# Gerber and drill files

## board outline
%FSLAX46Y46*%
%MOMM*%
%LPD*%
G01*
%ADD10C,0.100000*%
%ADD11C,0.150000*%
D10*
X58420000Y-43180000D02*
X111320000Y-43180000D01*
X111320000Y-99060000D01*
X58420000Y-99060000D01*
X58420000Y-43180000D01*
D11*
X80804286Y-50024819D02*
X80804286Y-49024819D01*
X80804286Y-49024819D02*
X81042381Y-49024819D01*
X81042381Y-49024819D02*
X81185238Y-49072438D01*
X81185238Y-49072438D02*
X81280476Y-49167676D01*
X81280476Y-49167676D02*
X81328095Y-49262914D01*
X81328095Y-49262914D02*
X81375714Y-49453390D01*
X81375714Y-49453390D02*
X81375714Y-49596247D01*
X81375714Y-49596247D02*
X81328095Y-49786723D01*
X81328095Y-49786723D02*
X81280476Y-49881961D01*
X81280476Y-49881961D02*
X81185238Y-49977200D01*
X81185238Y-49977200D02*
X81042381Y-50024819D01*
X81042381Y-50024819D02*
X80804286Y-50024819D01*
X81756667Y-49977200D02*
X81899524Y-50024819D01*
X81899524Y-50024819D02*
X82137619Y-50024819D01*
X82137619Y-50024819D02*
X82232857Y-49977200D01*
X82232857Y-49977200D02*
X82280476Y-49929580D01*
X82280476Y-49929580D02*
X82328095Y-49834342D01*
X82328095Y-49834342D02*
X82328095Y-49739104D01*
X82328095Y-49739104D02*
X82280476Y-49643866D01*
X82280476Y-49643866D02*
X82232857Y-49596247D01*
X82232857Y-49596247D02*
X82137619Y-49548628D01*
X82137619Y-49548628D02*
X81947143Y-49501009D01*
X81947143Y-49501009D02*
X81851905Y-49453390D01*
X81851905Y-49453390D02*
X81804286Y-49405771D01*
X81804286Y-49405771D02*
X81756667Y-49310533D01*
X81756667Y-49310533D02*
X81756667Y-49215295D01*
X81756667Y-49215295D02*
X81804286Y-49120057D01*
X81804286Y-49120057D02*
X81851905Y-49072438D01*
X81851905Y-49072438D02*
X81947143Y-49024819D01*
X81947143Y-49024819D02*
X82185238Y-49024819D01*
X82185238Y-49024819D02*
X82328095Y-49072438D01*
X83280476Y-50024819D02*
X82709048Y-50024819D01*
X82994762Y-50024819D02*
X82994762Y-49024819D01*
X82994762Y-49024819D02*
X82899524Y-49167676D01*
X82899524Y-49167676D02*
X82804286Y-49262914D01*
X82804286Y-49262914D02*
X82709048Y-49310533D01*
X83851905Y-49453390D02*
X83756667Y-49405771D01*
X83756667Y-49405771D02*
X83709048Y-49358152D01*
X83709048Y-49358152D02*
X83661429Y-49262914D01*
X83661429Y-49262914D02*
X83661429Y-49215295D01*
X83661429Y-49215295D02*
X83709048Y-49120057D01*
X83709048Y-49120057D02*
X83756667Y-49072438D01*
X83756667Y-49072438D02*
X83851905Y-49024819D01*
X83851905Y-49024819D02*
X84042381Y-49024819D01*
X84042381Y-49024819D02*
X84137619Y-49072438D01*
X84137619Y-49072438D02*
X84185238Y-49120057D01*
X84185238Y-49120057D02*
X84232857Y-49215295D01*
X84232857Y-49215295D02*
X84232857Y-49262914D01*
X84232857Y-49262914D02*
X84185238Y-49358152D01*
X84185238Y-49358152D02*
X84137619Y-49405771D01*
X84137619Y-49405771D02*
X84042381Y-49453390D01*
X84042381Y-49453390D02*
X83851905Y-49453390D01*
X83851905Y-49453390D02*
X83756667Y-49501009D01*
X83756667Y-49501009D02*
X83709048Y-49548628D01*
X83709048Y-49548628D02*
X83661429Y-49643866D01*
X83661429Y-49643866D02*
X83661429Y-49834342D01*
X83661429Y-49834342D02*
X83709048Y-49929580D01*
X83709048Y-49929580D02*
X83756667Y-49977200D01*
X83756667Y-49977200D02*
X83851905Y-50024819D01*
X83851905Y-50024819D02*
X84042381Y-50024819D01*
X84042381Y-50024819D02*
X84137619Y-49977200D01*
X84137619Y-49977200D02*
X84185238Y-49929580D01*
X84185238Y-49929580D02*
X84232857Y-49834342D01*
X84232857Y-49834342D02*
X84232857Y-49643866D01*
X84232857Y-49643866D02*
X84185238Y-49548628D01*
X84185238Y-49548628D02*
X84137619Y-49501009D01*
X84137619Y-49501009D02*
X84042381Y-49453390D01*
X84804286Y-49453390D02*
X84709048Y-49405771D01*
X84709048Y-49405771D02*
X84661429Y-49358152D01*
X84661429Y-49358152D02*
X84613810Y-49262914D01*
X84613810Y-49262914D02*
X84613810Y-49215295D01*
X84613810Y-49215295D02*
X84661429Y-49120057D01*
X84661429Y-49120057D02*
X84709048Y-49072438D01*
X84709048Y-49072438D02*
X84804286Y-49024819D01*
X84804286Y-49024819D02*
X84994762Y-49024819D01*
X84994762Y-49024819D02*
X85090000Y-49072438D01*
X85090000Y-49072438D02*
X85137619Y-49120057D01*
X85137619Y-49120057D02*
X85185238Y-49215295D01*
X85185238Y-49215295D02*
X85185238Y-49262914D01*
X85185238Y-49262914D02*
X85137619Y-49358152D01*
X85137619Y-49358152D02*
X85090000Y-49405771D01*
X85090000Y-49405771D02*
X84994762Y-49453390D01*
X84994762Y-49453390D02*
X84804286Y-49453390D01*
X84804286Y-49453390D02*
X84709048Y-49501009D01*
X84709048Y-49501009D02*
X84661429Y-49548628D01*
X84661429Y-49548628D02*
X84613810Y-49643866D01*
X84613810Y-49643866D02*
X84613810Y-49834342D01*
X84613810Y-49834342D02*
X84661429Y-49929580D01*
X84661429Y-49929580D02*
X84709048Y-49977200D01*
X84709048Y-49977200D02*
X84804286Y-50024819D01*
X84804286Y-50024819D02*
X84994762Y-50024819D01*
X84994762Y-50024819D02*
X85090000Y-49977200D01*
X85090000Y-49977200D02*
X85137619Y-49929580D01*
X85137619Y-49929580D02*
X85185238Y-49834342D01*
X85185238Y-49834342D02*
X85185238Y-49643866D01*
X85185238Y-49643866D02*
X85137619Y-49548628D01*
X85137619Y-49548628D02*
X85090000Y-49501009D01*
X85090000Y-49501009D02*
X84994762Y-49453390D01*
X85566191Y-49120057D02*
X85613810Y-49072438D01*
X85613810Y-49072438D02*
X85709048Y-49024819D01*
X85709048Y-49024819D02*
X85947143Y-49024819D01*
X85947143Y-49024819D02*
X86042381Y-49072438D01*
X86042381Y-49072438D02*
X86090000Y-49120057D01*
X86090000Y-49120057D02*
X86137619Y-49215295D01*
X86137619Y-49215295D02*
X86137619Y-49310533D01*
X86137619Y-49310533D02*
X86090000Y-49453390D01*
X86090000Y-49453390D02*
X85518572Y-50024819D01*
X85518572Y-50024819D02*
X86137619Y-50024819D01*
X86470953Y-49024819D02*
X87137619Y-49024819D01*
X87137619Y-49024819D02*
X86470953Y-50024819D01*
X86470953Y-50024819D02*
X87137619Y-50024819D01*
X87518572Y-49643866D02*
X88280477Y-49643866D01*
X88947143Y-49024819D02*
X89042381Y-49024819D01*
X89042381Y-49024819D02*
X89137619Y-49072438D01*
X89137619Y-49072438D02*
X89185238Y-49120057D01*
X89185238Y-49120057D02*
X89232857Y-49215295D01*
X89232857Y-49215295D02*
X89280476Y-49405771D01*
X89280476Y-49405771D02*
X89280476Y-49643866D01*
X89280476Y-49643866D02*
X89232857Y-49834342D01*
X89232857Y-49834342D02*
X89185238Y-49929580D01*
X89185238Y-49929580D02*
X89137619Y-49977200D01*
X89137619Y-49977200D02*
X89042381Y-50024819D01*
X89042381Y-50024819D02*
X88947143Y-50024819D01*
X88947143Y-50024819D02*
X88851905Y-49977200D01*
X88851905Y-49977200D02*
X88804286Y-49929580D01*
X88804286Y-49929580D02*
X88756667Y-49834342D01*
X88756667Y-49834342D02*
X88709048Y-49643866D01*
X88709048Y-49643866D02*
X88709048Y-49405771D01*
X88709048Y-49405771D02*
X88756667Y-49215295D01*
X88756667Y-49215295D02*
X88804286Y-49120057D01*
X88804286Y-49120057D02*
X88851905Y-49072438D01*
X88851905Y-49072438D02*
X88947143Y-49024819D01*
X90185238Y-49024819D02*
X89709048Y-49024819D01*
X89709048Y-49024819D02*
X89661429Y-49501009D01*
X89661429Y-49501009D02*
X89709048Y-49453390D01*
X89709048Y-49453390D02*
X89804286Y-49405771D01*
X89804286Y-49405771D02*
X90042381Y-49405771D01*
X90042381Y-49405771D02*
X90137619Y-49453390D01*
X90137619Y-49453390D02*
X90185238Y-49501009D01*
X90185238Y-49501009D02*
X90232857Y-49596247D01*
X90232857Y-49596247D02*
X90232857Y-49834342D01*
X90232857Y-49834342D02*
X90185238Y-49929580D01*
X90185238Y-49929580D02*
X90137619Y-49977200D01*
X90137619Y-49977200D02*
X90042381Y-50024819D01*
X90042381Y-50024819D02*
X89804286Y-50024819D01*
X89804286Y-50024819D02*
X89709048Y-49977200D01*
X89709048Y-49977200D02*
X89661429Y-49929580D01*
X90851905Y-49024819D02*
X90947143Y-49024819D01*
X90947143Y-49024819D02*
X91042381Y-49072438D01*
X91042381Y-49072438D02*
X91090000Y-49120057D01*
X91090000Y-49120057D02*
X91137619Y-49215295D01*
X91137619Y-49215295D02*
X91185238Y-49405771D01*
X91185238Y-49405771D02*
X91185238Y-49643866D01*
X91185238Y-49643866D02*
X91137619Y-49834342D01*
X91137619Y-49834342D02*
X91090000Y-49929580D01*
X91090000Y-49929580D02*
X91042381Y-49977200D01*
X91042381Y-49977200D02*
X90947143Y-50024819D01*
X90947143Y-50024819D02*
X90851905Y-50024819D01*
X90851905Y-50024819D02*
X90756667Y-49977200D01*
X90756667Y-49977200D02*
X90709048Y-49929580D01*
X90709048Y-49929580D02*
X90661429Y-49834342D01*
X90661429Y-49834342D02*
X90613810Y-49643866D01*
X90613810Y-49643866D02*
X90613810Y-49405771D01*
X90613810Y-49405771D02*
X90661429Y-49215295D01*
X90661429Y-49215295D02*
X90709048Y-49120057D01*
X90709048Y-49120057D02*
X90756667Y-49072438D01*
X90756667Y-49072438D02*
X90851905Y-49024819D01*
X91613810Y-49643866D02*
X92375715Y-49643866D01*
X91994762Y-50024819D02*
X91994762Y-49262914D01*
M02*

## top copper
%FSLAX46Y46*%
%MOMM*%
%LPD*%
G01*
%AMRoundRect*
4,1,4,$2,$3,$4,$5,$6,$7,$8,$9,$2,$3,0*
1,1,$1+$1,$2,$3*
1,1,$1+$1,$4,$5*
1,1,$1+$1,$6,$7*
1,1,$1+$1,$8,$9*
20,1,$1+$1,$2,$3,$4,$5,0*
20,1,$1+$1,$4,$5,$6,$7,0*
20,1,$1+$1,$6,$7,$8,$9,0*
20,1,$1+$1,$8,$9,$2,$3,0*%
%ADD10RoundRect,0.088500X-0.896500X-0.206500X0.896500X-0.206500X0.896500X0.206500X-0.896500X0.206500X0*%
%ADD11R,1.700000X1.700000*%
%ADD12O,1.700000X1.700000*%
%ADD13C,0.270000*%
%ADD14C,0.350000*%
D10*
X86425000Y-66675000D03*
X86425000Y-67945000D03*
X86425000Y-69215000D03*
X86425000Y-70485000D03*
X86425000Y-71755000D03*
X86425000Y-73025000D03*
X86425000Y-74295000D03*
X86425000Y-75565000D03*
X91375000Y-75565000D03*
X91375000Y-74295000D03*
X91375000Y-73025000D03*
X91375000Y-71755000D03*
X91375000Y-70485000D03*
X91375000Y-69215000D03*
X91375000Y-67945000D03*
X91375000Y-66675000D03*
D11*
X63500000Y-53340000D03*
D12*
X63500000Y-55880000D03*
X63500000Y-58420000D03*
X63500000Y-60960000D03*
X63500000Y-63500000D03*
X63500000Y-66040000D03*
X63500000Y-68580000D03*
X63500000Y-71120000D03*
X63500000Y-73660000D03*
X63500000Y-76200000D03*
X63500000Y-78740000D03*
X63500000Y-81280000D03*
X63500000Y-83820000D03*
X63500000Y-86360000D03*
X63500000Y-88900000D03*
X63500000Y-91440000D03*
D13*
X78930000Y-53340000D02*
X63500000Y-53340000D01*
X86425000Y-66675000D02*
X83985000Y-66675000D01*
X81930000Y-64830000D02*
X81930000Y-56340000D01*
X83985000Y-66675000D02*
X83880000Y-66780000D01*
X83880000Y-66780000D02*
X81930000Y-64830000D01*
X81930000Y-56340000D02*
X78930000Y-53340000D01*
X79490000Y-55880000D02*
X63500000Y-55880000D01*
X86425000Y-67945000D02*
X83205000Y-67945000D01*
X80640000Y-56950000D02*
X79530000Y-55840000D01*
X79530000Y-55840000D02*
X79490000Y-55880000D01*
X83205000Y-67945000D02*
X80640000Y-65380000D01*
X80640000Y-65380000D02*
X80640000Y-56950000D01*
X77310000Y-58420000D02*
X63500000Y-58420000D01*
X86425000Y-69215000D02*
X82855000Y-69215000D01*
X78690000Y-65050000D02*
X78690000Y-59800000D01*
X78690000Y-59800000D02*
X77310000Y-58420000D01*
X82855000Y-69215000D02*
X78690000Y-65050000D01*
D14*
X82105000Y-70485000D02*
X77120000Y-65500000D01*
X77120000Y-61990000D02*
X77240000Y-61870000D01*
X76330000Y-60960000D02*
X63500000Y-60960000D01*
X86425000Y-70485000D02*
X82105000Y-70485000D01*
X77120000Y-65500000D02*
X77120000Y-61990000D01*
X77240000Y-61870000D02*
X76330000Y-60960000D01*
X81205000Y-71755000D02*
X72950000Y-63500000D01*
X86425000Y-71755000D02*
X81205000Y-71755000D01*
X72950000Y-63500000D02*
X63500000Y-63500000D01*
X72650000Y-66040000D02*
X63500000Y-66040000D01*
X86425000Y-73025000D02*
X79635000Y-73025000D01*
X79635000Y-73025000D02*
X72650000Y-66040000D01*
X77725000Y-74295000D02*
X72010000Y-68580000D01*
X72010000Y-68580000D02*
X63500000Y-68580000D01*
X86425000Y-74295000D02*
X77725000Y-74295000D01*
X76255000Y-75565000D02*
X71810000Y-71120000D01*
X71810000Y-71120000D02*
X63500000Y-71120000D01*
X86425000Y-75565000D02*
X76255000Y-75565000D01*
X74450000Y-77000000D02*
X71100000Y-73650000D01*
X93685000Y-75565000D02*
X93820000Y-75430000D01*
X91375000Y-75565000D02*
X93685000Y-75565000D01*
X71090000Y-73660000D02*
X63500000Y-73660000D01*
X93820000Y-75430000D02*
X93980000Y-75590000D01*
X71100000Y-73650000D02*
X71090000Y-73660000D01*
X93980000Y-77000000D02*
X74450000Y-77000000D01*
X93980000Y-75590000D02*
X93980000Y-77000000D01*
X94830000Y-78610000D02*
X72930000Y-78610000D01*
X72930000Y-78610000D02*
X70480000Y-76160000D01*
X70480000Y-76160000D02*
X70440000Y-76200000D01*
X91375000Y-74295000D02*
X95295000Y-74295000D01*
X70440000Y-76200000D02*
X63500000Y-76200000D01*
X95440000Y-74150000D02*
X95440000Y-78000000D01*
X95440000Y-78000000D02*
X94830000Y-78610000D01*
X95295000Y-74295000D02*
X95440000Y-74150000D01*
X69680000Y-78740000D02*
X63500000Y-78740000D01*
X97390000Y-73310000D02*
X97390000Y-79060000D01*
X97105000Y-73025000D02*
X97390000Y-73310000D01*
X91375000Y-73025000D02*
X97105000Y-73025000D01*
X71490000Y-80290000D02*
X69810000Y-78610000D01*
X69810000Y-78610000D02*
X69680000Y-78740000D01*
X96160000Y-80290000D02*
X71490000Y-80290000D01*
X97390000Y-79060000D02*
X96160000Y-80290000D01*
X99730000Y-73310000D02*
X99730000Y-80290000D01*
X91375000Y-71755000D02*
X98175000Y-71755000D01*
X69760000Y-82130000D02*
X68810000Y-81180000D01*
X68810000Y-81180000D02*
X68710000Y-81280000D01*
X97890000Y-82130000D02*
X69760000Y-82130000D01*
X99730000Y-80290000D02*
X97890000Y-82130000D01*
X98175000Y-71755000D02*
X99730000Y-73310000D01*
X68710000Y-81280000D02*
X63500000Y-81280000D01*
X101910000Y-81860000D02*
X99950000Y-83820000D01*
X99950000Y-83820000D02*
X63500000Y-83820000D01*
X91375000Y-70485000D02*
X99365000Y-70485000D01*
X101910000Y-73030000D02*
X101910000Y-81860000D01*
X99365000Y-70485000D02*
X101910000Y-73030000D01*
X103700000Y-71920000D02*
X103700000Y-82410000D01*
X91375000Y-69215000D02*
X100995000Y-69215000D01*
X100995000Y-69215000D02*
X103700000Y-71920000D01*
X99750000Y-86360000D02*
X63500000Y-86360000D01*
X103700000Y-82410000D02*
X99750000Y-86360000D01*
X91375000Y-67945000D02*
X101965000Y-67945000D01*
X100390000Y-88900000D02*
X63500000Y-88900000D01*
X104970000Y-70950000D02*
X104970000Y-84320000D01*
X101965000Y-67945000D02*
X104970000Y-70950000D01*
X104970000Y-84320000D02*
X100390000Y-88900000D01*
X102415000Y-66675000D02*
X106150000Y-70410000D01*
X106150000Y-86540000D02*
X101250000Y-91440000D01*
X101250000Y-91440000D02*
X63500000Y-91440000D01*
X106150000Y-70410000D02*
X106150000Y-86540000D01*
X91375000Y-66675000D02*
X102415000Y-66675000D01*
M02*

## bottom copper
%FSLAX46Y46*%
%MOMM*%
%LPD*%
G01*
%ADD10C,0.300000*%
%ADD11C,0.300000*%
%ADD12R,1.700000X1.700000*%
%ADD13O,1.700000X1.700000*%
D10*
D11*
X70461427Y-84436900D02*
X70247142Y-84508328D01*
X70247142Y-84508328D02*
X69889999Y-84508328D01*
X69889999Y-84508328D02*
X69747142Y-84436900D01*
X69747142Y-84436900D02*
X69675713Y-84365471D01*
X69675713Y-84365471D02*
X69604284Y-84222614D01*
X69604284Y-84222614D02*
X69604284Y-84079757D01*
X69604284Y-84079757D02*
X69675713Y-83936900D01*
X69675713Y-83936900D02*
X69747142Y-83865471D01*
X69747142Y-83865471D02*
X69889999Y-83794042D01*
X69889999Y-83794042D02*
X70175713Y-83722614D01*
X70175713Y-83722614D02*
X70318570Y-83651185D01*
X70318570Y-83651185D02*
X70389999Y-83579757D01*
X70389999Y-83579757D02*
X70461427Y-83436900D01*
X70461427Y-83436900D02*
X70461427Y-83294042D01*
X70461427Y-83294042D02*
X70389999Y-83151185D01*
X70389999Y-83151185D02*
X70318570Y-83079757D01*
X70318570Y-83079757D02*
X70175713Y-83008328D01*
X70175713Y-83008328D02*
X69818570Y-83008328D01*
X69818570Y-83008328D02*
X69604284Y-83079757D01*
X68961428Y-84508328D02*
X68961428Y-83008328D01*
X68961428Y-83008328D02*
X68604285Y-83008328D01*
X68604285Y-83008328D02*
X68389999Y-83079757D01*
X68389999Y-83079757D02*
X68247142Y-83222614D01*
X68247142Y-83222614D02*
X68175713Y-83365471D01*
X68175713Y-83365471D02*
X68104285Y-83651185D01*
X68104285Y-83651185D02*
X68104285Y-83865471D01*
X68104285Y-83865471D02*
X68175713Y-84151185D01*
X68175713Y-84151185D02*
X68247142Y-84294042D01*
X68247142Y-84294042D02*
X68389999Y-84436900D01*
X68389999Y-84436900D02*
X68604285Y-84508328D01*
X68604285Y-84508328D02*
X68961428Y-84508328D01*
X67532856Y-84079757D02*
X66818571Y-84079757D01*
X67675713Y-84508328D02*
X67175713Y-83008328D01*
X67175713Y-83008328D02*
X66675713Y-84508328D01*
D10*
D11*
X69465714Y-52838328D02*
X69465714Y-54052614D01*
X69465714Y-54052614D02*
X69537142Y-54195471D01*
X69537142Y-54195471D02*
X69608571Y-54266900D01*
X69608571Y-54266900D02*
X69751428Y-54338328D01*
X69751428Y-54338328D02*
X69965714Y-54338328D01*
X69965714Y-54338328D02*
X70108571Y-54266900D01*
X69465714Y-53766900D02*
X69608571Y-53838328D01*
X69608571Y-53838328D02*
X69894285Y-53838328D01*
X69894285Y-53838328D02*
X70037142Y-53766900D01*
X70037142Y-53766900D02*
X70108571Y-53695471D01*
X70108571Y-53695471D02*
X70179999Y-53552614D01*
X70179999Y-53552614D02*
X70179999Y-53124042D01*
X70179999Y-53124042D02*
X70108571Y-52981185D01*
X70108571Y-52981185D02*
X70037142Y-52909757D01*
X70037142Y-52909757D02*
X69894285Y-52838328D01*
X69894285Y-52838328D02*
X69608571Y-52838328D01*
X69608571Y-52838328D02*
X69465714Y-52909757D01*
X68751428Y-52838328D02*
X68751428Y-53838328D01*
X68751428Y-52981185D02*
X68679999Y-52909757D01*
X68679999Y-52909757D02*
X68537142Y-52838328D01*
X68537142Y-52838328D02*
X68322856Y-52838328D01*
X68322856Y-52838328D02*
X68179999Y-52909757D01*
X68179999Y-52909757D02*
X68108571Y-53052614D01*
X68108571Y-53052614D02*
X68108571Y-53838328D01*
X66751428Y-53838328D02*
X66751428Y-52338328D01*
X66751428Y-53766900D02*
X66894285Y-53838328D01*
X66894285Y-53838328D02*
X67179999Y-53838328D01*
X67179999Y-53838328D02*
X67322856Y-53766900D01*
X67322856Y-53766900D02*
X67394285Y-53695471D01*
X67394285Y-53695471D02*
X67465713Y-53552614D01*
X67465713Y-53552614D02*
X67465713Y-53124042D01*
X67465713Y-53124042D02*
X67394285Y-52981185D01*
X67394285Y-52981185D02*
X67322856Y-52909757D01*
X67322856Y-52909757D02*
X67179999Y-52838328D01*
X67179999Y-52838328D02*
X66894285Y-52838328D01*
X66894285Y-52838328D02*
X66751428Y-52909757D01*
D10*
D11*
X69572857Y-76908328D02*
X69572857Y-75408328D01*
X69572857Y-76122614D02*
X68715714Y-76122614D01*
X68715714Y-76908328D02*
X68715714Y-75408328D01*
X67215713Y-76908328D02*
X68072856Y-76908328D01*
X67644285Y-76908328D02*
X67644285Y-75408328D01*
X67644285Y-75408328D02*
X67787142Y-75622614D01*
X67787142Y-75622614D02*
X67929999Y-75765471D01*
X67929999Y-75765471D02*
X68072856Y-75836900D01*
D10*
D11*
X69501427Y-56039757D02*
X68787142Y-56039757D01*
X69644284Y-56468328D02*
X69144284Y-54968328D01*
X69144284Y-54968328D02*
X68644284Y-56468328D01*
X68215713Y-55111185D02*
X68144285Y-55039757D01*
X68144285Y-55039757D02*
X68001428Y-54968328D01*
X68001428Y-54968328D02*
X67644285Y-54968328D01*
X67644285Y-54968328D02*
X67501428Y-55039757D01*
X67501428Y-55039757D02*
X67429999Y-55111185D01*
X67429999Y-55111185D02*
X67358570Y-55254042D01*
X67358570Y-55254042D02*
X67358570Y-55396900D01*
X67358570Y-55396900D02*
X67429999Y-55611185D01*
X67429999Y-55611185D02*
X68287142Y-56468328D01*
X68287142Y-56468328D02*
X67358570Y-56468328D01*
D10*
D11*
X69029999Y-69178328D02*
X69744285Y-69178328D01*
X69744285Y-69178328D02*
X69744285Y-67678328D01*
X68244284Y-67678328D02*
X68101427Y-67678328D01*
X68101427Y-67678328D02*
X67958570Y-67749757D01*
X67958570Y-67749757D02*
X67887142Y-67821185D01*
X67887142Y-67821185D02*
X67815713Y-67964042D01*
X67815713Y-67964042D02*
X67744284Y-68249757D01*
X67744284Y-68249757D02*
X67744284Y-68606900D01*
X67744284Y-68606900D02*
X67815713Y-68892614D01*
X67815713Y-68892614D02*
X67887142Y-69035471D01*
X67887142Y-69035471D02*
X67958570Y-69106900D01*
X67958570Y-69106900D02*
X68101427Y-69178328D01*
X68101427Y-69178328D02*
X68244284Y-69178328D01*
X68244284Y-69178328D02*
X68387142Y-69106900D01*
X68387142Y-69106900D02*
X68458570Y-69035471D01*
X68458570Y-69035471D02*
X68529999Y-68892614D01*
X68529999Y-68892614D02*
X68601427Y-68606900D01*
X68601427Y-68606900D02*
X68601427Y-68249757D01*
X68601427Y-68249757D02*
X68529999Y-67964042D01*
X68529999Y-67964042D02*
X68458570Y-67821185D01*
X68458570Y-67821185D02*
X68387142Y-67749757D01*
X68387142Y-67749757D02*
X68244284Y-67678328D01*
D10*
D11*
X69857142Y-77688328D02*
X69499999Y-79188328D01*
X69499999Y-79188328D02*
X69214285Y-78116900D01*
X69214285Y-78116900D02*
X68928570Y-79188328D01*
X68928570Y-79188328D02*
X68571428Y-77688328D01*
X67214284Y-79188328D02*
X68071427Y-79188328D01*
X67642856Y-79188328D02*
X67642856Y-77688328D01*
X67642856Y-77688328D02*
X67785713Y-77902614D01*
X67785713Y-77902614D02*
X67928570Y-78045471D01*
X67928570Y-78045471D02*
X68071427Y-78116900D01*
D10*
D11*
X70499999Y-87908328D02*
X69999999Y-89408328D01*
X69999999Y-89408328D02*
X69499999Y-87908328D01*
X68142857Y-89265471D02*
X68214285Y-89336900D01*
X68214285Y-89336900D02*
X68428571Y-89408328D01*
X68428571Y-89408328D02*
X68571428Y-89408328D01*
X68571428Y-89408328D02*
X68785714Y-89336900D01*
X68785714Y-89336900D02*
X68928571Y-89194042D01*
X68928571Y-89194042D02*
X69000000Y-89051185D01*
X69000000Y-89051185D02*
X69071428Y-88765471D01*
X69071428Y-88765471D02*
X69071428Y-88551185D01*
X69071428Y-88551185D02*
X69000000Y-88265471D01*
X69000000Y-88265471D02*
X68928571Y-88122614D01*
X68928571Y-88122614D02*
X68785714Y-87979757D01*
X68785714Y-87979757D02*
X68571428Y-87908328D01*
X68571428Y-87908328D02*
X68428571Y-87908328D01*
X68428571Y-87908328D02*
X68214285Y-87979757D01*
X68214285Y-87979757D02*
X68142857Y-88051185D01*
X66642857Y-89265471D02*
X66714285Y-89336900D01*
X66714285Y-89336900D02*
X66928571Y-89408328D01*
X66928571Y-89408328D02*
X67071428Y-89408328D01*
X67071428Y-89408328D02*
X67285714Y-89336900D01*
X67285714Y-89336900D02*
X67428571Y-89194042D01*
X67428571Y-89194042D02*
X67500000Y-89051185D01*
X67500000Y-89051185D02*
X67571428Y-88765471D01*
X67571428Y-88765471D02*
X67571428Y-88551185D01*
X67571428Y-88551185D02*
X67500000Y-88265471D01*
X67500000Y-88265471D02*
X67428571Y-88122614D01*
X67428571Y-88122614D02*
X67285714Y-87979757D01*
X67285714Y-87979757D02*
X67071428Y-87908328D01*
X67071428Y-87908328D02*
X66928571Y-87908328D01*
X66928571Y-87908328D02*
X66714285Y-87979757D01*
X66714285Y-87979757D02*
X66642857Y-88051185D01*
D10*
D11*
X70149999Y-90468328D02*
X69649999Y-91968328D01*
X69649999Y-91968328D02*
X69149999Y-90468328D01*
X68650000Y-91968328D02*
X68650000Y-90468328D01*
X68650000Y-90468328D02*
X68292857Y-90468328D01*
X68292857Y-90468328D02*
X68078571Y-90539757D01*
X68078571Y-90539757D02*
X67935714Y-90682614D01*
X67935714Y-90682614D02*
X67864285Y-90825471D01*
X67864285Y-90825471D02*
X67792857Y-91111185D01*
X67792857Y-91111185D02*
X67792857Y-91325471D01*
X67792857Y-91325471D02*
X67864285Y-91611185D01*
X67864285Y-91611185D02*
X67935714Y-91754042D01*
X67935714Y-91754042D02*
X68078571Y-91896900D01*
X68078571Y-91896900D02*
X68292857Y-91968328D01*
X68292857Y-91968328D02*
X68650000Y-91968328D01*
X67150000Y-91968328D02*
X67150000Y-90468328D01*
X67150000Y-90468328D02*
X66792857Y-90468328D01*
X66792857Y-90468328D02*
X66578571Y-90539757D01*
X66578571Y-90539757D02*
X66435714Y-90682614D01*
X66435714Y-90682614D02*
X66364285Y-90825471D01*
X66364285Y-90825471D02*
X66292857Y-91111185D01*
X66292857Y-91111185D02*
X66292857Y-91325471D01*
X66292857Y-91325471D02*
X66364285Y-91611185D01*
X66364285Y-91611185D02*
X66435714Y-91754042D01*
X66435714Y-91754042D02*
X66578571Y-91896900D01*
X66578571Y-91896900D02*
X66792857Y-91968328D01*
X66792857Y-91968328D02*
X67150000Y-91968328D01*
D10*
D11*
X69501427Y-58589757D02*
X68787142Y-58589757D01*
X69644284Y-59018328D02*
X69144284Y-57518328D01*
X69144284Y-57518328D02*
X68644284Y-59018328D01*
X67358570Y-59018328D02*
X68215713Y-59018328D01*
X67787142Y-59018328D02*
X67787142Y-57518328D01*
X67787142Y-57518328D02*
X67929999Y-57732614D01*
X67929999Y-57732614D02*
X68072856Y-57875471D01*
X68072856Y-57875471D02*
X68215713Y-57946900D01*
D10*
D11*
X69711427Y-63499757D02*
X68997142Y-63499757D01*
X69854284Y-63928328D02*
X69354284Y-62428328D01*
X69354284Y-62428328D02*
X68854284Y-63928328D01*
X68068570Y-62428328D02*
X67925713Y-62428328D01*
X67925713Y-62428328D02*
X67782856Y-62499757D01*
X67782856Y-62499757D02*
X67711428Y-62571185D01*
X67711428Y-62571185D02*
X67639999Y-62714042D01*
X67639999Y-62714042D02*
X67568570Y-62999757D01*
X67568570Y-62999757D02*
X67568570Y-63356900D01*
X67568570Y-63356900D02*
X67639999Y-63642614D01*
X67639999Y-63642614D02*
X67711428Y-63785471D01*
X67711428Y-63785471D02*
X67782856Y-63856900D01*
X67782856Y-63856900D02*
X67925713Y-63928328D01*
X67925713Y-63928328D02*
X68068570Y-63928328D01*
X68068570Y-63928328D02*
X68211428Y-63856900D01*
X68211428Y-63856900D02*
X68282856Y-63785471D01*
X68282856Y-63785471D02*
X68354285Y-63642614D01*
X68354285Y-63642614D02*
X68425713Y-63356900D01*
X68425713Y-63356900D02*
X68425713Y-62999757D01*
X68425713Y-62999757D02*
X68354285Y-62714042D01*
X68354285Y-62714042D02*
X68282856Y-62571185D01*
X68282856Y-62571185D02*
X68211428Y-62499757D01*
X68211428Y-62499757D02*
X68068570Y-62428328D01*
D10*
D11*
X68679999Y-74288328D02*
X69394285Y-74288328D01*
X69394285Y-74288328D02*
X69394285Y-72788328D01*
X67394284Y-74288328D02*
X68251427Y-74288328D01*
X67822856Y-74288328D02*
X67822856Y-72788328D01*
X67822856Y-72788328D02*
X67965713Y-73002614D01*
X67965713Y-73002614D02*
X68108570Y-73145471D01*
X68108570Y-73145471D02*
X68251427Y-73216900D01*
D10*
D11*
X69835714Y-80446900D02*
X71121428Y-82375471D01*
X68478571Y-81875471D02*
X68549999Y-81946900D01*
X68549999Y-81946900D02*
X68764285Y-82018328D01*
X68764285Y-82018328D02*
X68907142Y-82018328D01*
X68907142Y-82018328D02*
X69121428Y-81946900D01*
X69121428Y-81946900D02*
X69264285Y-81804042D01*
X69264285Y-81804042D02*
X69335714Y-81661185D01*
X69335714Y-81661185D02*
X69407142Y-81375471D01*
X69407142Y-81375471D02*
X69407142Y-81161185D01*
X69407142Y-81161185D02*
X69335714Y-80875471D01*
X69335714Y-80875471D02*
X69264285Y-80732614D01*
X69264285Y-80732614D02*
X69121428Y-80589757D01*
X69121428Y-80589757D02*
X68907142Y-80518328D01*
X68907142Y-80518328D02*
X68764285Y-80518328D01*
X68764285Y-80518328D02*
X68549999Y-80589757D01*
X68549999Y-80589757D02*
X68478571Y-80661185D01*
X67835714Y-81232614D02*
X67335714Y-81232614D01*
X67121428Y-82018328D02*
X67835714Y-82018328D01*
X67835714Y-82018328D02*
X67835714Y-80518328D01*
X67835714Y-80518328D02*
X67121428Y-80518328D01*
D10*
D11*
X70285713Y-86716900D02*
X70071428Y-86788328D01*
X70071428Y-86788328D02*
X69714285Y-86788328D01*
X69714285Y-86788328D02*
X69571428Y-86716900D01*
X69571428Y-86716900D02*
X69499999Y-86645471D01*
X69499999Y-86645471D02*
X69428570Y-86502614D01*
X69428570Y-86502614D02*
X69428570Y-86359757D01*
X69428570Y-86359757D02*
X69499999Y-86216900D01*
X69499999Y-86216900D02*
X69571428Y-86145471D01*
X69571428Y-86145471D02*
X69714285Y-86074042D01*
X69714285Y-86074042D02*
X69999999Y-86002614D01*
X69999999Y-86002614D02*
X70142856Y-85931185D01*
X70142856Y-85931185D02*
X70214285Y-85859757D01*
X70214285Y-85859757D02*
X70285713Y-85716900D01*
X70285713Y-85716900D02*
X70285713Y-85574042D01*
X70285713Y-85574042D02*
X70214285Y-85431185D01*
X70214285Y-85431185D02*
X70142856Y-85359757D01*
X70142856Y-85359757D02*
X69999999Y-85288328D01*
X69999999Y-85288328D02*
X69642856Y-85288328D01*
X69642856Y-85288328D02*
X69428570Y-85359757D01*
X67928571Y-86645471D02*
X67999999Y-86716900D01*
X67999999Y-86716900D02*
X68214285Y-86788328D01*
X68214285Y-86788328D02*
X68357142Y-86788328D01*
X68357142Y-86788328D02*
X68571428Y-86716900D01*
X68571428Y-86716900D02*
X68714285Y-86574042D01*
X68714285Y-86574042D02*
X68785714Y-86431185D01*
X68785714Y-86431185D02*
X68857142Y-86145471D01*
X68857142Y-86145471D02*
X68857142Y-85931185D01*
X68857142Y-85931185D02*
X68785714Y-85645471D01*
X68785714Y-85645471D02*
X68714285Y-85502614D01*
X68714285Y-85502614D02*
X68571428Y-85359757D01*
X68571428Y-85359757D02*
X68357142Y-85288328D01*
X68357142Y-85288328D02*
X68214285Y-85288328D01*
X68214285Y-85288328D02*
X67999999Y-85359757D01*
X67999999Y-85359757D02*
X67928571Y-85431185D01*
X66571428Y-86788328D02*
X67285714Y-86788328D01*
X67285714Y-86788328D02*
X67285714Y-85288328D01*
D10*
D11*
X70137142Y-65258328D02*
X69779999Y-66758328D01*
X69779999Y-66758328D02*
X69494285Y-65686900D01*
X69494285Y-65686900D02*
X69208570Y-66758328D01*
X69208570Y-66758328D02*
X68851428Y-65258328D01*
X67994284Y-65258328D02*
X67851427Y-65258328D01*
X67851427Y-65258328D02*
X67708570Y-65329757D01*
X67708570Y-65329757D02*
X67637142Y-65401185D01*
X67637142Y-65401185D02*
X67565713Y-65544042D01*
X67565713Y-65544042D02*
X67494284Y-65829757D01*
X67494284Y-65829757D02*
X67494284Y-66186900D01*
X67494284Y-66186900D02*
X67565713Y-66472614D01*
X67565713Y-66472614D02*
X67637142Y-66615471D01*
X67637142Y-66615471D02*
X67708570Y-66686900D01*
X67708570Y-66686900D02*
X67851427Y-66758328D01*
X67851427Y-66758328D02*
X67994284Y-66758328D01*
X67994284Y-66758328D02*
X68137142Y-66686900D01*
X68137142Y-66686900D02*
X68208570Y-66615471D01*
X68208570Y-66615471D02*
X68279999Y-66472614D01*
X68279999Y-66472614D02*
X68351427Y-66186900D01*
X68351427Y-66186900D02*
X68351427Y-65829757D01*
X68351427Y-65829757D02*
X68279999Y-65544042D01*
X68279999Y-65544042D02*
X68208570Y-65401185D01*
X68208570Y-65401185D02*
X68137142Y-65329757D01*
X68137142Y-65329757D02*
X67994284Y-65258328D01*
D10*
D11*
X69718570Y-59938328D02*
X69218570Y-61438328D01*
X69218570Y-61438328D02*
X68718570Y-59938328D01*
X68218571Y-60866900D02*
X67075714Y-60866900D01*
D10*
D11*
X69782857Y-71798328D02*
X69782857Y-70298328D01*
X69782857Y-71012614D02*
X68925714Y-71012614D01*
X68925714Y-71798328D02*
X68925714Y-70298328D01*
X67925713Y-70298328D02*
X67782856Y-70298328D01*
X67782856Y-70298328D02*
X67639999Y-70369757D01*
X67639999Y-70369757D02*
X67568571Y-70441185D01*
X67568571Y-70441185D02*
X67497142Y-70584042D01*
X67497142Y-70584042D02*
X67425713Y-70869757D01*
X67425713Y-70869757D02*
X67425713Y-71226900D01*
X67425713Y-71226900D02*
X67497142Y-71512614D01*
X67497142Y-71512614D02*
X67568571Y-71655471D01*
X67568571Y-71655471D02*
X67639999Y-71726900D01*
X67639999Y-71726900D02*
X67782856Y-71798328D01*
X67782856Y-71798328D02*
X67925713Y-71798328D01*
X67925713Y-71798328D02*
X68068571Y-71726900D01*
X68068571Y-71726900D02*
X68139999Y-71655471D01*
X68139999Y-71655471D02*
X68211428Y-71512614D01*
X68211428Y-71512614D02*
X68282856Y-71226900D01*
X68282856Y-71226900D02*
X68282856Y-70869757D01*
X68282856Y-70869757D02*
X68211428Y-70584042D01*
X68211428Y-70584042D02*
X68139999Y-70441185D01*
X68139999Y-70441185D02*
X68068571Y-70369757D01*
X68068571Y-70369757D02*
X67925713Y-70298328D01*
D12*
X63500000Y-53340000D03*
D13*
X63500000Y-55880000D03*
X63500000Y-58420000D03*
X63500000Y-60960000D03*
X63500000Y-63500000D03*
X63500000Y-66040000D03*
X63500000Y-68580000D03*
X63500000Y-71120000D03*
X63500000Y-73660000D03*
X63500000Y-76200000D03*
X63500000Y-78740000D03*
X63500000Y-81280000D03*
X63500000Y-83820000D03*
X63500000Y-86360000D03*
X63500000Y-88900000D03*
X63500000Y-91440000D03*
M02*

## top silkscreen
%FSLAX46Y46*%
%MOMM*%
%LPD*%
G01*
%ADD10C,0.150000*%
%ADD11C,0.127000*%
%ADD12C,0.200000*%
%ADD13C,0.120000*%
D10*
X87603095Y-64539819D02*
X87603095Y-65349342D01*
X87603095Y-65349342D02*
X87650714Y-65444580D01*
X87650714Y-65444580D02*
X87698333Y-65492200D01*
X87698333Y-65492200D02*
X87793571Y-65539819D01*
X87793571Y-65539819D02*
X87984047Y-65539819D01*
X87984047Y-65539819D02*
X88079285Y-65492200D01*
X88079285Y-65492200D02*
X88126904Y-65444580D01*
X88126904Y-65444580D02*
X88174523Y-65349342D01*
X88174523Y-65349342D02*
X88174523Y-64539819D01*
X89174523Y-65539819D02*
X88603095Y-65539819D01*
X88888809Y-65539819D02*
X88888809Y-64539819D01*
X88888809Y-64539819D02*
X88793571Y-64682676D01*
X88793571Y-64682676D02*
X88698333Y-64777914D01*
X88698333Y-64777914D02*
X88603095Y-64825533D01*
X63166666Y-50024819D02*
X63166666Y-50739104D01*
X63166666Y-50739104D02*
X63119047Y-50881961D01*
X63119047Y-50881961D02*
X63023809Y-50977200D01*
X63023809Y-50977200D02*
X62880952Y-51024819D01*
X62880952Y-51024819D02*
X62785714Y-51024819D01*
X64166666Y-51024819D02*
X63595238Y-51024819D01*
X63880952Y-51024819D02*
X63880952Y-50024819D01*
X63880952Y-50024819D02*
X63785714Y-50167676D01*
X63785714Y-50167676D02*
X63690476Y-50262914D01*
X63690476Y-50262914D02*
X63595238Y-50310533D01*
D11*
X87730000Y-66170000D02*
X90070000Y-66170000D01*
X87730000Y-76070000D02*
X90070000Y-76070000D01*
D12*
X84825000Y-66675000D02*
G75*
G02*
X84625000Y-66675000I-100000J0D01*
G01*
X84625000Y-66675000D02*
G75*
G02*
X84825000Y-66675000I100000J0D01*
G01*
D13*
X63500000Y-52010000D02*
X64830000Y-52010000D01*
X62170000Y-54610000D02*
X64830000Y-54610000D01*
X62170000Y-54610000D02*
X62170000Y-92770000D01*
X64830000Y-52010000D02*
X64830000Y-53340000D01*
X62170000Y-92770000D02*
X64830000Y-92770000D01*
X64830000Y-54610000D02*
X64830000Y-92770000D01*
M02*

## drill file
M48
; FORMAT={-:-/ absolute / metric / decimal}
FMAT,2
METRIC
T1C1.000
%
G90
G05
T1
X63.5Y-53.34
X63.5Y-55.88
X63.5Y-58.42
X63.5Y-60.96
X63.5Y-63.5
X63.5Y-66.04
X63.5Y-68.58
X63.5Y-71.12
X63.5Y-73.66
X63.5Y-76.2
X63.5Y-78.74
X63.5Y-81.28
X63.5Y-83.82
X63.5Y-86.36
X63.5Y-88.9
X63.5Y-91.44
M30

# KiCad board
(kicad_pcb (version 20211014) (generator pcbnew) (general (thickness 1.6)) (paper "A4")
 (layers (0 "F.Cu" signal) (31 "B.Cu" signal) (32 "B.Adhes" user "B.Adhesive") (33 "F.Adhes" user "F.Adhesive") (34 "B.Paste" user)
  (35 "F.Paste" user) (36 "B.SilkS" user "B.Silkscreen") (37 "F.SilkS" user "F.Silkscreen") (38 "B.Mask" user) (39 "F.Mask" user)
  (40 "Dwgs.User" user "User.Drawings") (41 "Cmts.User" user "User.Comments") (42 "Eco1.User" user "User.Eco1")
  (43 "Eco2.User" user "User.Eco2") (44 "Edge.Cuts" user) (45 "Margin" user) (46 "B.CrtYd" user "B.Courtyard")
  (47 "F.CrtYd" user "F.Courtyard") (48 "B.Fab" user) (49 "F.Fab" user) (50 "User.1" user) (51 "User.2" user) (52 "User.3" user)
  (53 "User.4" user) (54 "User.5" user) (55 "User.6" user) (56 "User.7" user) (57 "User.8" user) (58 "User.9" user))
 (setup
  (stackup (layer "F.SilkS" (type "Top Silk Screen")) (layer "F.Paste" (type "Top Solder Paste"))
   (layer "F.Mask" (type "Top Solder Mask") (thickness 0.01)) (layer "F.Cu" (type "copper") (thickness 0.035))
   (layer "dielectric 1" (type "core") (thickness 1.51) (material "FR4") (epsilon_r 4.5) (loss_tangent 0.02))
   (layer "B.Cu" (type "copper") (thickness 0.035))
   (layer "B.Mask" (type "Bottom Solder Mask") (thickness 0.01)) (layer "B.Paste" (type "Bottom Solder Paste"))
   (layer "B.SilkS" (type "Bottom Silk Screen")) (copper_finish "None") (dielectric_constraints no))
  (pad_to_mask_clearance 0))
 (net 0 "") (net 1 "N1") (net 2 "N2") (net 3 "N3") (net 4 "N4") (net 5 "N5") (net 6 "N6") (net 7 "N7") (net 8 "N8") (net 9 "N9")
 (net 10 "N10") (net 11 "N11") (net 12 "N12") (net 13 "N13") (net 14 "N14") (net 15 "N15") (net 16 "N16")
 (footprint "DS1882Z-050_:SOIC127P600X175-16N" (layer "F.Cu") (at 88.9 71.12)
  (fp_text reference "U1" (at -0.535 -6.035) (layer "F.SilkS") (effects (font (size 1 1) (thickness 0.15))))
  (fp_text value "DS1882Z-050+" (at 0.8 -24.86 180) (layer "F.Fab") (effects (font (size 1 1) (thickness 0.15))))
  (fp_line (start -1.17 -4.95) (end 1.17 -4.95) (layer "F.SilkS") (width 0.127))
  (fp_line (start -1.17 4.95) (end 1.17 4.95) (layer "F.SilkS") (width 0.127))
  (fp_circle (center -4.175 -4.445) (end -4.075 -4.445) (layer "F.SilkS") (width 0.2) (fill none))
  (pad "1" smd roundrect (at -2.475 -4.445) (size 1.97 0.59) (layers "F.Cu" "F.Paste" "F.Mask") (roundrect_rratio 0.15) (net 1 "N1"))
  (pad "2" smd roundrect (at -2.475 -3.175) (size 1.97 0.59) (layers "F.Cu" "F.Paste" "F.Mask") (roundrect_rratio 0.15) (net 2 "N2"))
  (pad "3" smd roundrect (at -2.475 -1.905) (size 1.97 0.59) (layers "F.Cu" "F.Paste" "F.Mask") (roundrect_rratio 0.15) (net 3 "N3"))
  (pad "4" smd roundrect (at -2.475 -0.635) (size 1.97 0.59) (layers "F.Cu" "F.Paste" "F.Mask") (roundrect_rratio 0.15) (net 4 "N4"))
  (pad "5" smd roundrect (at -2.475 0.635) (size 1.97 0.59) (layers "F.Cu" "F.Paste" "F.Mask") (roundrect_rratio 0.15) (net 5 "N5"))
  (pad "6" smd roundrect (at -2.475 1.905) (size 1.97 0.59) (layers "F.Cu" "F.Paste" "F.Mask") (roundrect_rratio 0.15) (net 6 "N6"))
  (pad "7" smd roundrect (at -2.475 3.175) (size 1.97 0.59) (layers "F.Cu" "F.Paste" "F.Mask") (roundrect_rratio 0.15) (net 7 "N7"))
  (pad "8" smd roundrect (at -2.475 4.445) (size 1.97 0.59) (layers "F.Cu" "F.Paste" "F.Mask") (roundrect_rratio 0.15) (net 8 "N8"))
  (pad "9" smd roundrect (at 2.475 4.445) (size 1.97 0.59) (layers "F.Cu" "F.Paste" "F.Mask") (roundrect_rratio 0.15) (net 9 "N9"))
  (pad "10" smd roundrect (at 2.475 3.175) (size 1.97 0.59) (layers "F.Cu" "F.Paste" "F.Mask") (roundrect_rratio 0.15) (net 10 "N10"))
  (pad "11" smd roundrect (at 2.475 1.905) (size 1.97 0.59) (layers "F.Cu" "F.Paste" "F.Mask") (roundrect_rratio 0.15) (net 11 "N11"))
  (pad "12" smd roundrect (at 2.475 0.635) (size 1.97 0.59) (layers "F.Cu" "F.Paste" "F.Mask") (roundrect_rratio 0.15) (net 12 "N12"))
  (pad "13" smd roundrect (at 2.475 -0.635) (size 1.97 0.59) (layers "F.Cu" "F.Paste" "F.Mask") (roundrect_rratio 0.15) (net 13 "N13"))
  (pad "14" smd roundrect (at 2.475 -1.905) (size 1.97 0.59) (layers "F.Cu" "F.Paste" "F.Mask") (roundrect_rratio 0.15) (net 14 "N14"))
  (pad "15" smd roundrect (at 2.475 -3.175) (size 1.97 0.59) (layers "F.Cu" "F.Paste" "F.Mask") (roundrect_rratio 0.15) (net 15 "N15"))
  (pad "16" smd roundrect (at 2.475 -4.445) (size 1.97 0.59) (layers "F.Cu" "F.Paste" "F.Mask") (roundrect_rratio 0.15) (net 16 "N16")))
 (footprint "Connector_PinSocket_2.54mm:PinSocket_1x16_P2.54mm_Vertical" (layer "F.Cu") (at 63.5 53.34)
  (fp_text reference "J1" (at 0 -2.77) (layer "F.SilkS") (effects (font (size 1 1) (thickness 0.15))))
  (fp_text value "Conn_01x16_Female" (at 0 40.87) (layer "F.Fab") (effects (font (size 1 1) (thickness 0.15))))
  (fp_line (start 0 -1.33) (end 1.33 -1.33) (layer "F.SilkS") (width 0.12))
  (fp_line (start -1.33 1.27) (end 1.33 1.27) (layer "F.SilkS") (width 0.12))
  (fp_line (start -1.33 1.27) (end -1.33 39.43) (layer "F.SilkS") (width 0.12))
  (fp_line (start 1.33 -1.33) (end 1.33 0) (layer "F.SilkS") (width 0.12))
  (fp_line (start -1.33 39.43) (end 1.33 39.43) (layer "F.SilkS") (width 0.12))
  (fp_line (start 1.33 1.27) (end 1.33 39.43) (layer "F.SilkS") (width 0.12))
  (pad "1" thru_hole rect (at 0 0) (size 1.7 1.7) (drill 1) (layers *.Cu *.Mask) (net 1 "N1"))
  (pad "2" thru_hole oval (at 0 2.54) (size 1.7 1.7) (drill 1) (layers *.Cu *.Mask) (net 2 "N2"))
  (pad "3" thru_hole oval (at 0 5.08) (size 1.7 1.7) (drill 1) (layers *.Cu *.Mask) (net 3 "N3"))
  (pad "4" thru_hole oval (at 0 7.62) (size 1.7 1.7) (drill 1) (layers *.Cu *.Mask) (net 4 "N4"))
  (pad "5" thru_hole oval (at 0 10.16) (size 1.7 1.7) (drill 1) (layers *.Cu *.Mask) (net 5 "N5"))
  (pad "6" thru_hole oval (at 0 12.7) (size 1.7 1.7) (drill 1) (layers *.Cu *.Mask) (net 6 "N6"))
  (pad "7" thru_hole oval (at 0 15.24) (size 1.7 1.7) (drill 1) (layers *.Cu *.Mask) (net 7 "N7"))
  (pad "8" thru_hole oval (at 0 17.78) (size 1.7 1.7) (drill 1) (layers *.Cu *.Mask) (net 8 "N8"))
  (pad "9" thru_hole oval (at 0 20.32) (size 1.7 1.7) (drill 1) (layers *.Cu *.Mask) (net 9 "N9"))
  (pad "10" thru_hole oval (at 0 22.86) (size 1.7 1.7) (drill 1) (layers *.Cu *.Mask) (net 10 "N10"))
  (pad "11" thru_hole oval (at 0 25.4) (size 1.7 1.7) (drill 1) (layers *.Cu *.Mask) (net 11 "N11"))
  (pad "12" thru_hole oval (at 0 27.94) (size 1.7 1.7) (drill 1) (layers *.Cu *.Mask) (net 12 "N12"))
  (pad "13" thru_hole oval (at 0 30.48) (size 1.7 1.7) (drill 1) (layers *.Cu *.Mask) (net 13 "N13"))
  (pad "14" thru_hole oval (at 0 33.02) (size 1.7 1.7) (drill 1) (layers *.Cu *.Mask) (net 14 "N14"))
  (pad "15" thru_hole oval (at 0 35.56) (size 1.7 1.7) (drill 1) (layers *.Cu *.Mask) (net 15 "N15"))
  (pad "16" thru_hole oval (at 0 38.1) (size 1.7 1.7) (drill 1) (layers *.Cu *.Mask) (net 16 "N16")))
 (gr_rect (start 58.42 43.18) (end 111.32 99.06) (layer "Edge.Cuts") (width 0.1) (fill none))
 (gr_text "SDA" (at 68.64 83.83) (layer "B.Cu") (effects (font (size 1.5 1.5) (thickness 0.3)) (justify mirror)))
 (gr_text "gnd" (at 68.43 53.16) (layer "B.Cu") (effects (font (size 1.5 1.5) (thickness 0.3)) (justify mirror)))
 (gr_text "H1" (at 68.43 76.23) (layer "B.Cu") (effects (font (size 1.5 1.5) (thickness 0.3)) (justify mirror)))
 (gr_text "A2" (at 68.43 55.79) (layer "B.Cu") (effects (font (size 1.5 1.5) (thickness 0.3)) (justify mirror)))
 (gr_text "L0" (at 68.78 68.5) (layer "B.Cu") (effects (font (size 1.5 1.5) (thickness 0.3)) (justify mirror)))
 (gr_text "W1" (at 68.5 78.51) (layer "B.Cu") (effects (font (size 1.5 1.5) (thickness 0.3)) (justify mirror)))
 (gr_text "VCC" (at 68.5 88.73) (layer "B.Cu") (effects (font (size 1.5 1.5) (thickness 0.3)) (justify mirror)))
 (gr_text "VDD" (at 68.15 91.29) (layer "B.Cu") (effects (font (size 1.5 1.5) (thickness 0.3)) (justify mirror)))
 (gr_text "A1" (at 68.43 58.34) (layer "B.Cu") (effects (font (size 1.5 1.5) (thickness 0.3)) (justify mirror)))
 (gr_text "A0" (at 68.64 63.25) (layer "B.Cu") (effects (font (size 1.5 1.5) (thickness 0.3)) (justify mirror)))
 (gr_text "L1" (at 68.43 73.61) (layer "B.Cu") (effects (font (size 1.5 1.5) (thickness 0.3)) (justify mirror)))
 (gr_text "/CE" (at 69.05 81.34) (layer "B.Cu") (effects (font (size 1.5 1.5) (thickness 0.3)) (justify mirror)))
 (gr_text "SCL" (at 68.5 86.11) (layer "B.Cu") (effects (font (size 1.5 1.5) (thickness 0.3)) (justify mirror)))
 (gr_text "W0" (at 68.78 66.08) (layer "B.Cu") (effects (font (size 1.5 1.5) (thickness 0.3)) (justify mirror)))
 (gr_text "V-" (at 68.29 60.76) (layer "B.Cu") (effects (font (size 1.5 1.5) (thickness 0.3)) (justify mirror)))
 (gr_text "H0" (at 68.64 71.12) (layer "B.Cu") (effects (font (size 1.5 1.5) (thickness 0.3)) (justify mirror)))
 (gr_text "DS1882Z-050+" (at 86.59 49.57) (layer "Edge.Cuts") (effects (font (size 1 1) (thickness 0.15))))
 (segment (start 78.93 53.34) (end 63.5 53.34) (width 0.27) (layer "F.Cu") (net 1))
 (segment (start 86.425 66.675) (end 83.985 66.675) (width 0.27) (layer "F.Cu") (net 1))
 (segment (start 81.93 64.83) (end 81.93 56.34) (width 0.27) (layer "F.Cu") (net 1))
 (segment (start 83.985 66.675) (end 83.88 66.78) (width 0.27) (layer "F.Cu") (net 1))
 (segment (start 83.88 66.78) (end 81.93 64.83) (width 0.27) (layer "F.Cu") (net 1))
 (segment (start 81.93 56.34) (end 78.93 53.34) (width 0.27) (layer "F.Cu") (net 1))
 (segment (start 79.49 55.88) (end 63.5 55.88) (width 0.27) (layer "F.Cu") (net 2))
 (segment (start 86.425 67.945) (end 83.205 67.945) (width 0.27) (layer "F.Cu") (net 2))
 (segment (start 80.64 56.95) (end 79.53 55.84) (width 0.27) (layer "F.Cu") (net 2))
 (segment (start 79.53 55.84) (end 79.49 55.88) (width 0.27) (layer "F.Cu") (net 2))
 (segment (start 83.205 67.945) (end 80.64 65.38) (width 0.27) (layer "F.Cu") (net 2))
 (segment (start 80.64 65.38) (end 80.64 56.95) (width 0.27) (layer "F.Cu") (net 2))
 (segment (start 77.31 58.42) (end 63.5 58.42) (width 0.27) (layer "F.Cu") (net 3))
 (segment (start 86.425 69.215) (end 82.855 69.215) (width 0.27) (layer "F.Cu") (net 3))
 (segment (start 78.69 65.05) (end 78.69 59.8) (width 0.27) (layer "F.Cu") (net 3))
 (segment (start 78.69 59.8) (end 77.31 58.42) (width 0.27) (layer "F.Cu") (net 3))
 (segment (start 82.855 69.215) (end 78.69 65.05) (width 0.27) (layer "F.Cu") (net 3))
 (segment (start 82.105 70.485) (end 77.12 65.5) (width 0.35) (layer "F.Cu") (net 4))
 (segment (start 77.12 61.99) (end 77.24 61.87) (width 0.35) (layer "F.Cu") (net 4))
 (segment (start 76.33 60.96) (end 63.5 60.96) (width 0.35) (layer "F.Cu") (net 4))
 (segment (start 86.425 70.485) (end 82.105 70.485) (width 0.35) (layer "F.Cu") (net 4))
 (segment (start 77.12 65.5) (end 77.12 61.99) (width 0.35) (layer "F.Cu") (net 4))
 (segment (start 77.24 61.87) (end 76.33 60.96) (width 0.35) (layer "F.Cu") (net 4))
 (segment (start 81.205 71.755) (end 72.95 63.5) (width 0.35) (layer "F.Cu") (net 5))
 (segment (start 86.425 71.755) (end 81.205 71.755) (width 0.35) (layer "F.Cu") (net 5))
 (segment (start 72.95 63.5) (end 63.5 63.5) (width 0.35) (layer "F.Cu") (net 5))
 (segment (start 72.65 66.04) (end 63.5 66.04) (width 0.35) (layer "F.Cu") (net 6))
 (segment (start 86.425 73.025) (end 79.635 73.025) (width 0.35) (layer "F.Cu") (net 6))
 (segment (start 79.635 73.025) (end 72.65 66.04) (width 0.35) (layer "F.Cu") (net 6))
 (segment (start 77.725 74.295) (end 72.01 68.58) (width 0.35) (layer "F.Cu") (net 7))
 (segment (start 72.01 68.58) (end 63.5 68.58) (width 0.35) (layer "F.Cu") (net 7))
 (segment (start 86.425 74.295) (end 77.725 74.295) (width 0.35) (layer "F.Cu") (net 7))
 (segment (start 76.255 75.565) (end 71.81 71.12) (width 0.35) (layer "F.Cu") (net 8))
 (segment (start 71.81 71.12) (end 63.5 71.12) (width 0.35) (layer "F.Cu") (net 8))
 (segment (start 86.425 75.565) (end 76.255 75.565) (width 0.35) (layer "F.Cu") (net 8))
 (segment (start 74.45 77) (end 71.1 73.65) (width 0.35) (layer "F.Cu") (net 9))
 (segment (start 93.685 75.565) (end 93.82 75.43) (width 0.35) (layer "F.Cu") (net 9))
 (segment (start 91.375 75.565) (end 93.685 75.565) (width 0.35) (layer "F.Cu") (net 9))
 (segment (start 71.09 73.66) (end 63.5 73.66) (width 0.35) (layer "F.Cu") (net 9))
 (segment (start 93.82 75.43) (end 93.98 75.59) (width 0.35) (layer "F.Cu") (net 9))
 (segment (start 71.1 73.65) (end 71.09 73.66) (width 0.35) (layer "F.Cu") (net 9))
 (segment (start 93.98 77) (end 74.45 77) (width 0.35) (layer "F.Cu") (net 9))
 (segment (start 93.98 75.59) (end 93.98 77) (width 0.35) (layer "F.Cu") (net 9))
 (segment (start 94.83 78.61) (end 72.93 78.61) (width 0.35) (layer "F.Cu") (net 10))
 (segment (start 72.93 78.61) (end 70.48 76.16) (width 0.35) (layer "F.Cu") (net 10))
 (segment (start 70.48 76.16) (end 70.44 76.2) (width 0.35) (layer "F.Cu") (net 10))
 (segment (start 91.375 74.295) (end 95.295 74.295) (width 0.35) (layer "F.Cu") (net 10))
 (segment (start 70.44 76.2) (end 63.5 76.2) (width 0.35) (layer "F.Cu") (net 10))
 (segment (start 95.44 74.15) (end 95.44 78) (width 0.35) (layer "F.Cu") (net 10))
 (segment (start 95.44 78) (end 94.83 78.61) (width 0.35) (layer "F.Cu") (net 10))
 (segment (start 95.295 74.295) (end 95.44 74.15) (width 0.35) (layer "F.Cu") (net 10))
 (segment (start 69.68 78.74) (end 63.5 78.74) (width 0.35) (layer "F.Cu") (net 11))
 (segment (start 97.39 73.31) (end 97.39 79.06) (width 0.35) (layer "F.Cu") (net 11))
 (segment (start 97.105 73.025) (end 97.39 73.31) (width 0.35) (layer "F.Cu") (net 11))
 (segment (start 91.375 73.025) (end 97.105 73.025) (width 0.35) (layer "F.Cu") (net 11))
 (segment (start 71.49 80.29) (end 69.81 78.61) (width 0.35) (layer "F.Cu") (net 11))
 (segment (start 69.81 78.61) (end 69.68 78.74) (width 0.35) (layer "F.Cu") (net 11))
 (segment (start 96.16 80.29) (end 71.49 80.29) (width 0.35) (layer "F.Cu") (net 11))
 (segment (start 97.39 79.06) (end 96.16 80.29) (width 0.35) (layer "F.Cu") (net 11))
 (segment (start 99.73 73.31) (end 99.73 80.29) (width 0.35) (layer "F.Cu") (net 12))
 (segment (start 91.375 71.755) (end 98.175 71.755) (width 0.35) (layer "F.Cu") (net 12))
 (segment (start 69.76 82.13) (end 68.81 81.18) (width 0.35) (layer "F.Cu") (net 12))
 (segment (start 68.81 81.18) (end 68.71 81.28) (width 0.35) (layer "F.Cu") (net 12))
 (segment (start 97.89 82.13) (end 69.76 82.13) (width 0.35) (layer "F.Cu") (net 12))
 (segment (start 99.73 80.29) (end 97.89 82.13) (width 0.35) (layer "F.Cu") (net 12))
 (segment (start 98.175 71.755) (end 99.73 73.31) (width 0.35) (layer "F.Cu") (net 12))
 (segment (start 68.71 81.28) (end 63.5 81.28) (width 0.35) (layer "F.Cu") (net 12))
 (segment (start 101.91 81.86) (end 99.95 83.82) (width 0.35) (layer "F.Cu") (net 13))
 (segment (start 99.95 83.82) (end 63.5 83.82) (width 0.35) (layer "F.Cu") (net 13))
 (segment (start 91.375 70.485) (end 99.365 70.485) (width 0.35) (layer "F.Cu") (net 13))
 (segment (start 101.91 73.03) (end 101.91 81.86) (width 0.35) (layer "F.Cu") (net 13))
 (segment (start 99.365 70.485) (end 101.91 73.03) (width 0.35) (layer "F.Cu") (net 13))
 (segment (start 103.7 71.92) (end 103.7 82.41) (width 0.35) (layer "F.Cu") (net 14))
 (segment (start 91.375 69.215) (end 100.995 69.215) (width 0.35) (layer "F.Cu") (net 14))
 (segment (start 100.995 69.215) (end 103.7 71.92) (width 0.35) (layer "F.Cu") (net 14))
 (segment (start 99.75 86.36) (end 63.5 86.36) (width 0.35) (layer "F.Cu") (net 14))
 (segment (start 103.7 82.41) (end 99.75 86.36) (width 0.35) (layer "F.Cu") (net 14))
 (segment (start 91.375 67.945) (end 101.965 67.945) (width 0.35) (layer "F.Cu") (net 15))
 (segment (start 100.39 88.9) (end 63.5 88.9) (width 0.35) (layer "F.Cu") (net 15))
 (segment (start 104.97 70.95) (end 104.97 84.32) (width 0.35) (layer "F.Cu") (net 15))
 (segment (start 101.965 67.945) (end 104.97 70.95) (width 0.35) (layer "F.Cu") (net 15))
 (segment (start 104.97 84.32) (end 100.39 88.9) (width 0.35) (layer "F.Cu") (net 15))
 (segment (start 102.415 66.675) (end 106.15 70.41) (width 0.35) (layer "F.Cu") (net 16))
 (segment (start 106.15 86.54) (end 101.25 91.44) (width 0.35) (layer "F.Cu") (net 16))
 (segment (start 101.25 91.44) (end 63.5 91.44) (width 0.35) (layer "F.Cu") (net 16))
 (segment (start 106.15 70.41) (end 106.15 86.54) (width 0.35) (layer "F.Cu") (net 16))
 (segment (start 91.375 66.675) (end 102.415 66.675) (width 0.35) (layer "F.Cu") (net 16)))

